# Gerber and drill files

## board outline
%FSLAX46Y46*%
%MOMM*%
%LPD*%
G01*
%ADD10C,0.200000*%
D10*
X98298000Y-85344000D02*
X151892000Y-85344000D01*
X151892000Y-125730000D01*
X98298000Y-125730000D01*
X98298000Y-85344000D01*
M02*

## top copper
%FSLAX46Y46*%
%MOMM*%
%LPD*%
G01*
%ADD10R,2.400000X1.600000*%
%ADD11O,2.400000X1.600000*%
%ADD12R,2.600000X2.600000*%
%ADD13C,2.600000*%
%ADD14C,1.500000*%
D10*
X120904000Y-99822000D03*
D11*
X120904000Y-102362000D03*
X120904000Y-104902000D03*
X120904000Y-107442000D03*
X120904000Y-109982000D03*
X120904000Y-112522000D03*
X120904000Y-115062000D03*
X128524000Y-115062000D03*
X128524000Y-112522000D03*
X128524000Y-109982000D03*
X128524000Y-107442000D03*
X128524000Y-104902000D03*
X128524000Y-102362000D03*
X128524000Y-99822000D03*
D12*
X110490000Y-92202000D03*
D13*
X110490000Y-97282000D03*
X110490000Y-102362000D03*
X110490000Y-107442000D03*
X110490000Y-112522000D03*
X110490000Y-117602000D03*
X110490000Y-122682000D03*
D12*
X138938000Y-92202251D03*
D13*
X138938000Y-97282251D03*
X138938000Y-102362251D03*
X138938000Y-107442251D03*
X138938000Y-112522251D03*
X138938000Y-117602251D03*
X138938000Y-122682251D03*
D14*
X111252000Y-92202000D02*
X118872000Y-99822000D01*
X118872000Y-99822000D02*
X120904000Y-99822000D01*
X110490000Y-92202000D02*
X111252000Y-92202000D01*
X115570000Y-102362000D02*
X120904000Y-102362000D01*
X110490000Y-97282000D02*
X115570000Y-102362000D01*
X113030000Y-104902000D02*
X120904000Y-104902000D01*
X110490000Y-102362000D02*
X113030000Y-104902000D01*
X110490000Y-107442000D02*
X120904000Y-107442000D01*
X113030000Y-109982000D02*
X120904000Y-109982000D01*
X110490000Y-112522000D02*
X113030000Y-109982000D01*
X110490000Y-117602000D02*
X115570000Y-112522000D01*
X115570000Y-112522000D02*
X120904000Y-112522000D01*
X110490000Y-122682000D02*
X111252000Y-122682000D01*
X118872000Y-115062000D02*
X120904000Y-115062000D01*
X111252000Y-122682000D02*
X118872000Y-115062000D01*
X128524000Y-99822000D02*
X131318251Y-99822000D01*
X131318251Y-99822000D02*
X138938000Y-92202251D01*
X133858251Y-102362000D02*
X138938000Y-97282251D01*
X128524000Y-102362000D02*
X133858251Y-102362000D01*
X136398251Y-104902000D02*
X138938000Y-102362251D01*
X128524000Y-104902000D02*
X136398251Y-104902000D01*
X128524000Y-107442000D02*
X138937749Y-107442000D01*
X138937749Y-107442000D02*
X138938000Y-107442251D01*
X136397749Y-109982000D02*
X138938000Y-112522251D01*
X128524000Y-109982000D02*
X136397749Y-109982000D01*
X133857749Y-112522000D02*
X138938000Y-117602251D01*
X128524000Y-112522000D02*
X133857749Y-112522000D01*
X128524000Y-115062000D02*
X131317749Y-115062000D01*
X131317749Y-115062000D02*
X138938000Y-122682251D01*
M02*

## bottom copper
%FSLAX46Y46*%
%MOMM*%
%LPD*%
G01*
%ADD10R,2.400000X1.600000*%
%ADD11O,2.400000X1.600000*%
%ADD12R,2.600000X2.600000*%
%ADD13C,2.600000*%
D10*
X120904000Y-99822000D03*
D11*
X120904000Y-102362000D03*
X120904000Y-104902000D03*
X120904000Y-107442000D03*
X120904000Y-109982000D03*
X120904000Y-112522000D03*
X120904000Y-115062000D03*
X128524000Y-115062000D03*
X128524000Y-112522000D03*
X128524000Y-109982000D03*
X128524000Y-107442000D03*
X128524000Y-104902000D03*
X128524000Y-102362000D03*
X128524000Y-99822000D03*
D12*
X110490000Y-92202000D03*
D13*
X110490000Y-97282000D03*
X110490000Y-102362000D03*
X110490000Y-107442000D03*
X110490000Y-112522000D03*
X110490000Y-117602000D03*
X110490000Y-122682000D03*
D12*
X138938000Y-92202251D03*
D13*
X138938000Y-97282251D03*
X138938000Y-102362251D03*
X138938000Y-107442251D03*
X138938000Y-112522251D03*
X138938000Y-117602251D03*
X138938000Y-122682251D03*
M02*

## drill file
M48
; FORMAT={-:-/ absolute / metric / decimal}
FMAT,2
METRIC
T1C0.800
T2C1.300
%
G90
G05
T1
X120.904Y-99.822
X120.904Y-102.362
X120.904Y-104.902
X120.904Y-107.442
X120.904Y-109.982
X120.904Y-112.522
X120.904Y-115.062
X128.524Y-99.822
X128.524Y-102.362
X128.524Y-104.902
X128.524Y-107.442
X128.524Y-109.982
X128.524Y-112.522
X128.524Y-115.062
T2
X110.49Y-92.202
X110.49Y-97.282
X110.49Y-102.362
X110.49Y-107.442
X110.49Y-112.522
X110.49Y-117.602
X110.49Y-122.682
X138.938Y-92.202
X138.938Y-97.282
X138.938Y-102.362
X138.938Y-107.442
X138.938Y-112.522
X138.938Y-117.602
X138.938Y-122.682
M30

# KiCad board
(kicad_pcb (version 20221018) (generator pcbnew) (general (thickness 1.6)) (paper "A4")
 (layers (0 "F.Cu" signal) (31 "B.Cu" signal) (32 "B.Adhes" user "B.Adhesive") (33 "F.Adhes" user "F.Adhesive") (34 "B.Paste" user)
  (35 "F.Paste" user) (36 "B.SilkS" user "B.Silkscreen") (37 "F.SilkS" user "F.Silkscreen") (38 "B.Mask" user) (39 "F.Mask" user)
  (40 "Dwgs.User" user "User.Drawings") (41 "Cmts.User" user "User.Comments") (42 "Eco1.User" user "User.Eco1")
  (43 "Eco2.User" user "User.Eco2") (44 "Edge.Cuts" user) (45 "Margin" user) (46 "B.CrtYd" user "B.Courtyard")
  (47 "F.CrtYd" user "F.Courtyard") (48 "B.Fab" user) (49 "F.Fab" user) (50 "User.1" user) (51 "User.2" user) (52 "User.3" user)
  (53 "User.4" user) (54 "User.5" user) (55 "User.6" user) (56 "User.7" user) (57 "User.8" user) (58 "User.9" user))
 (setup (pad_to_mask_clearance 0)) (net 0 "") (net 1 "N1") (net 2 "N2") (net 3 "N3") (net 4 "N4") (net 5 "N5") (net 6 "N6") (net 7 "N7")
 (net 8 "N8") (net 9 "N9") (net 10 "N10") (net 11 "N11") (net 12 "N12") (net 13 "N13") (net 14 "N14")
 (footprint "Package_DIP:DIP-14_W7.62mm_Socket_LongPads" (layer "F.Cu") (at 120.904 99.822)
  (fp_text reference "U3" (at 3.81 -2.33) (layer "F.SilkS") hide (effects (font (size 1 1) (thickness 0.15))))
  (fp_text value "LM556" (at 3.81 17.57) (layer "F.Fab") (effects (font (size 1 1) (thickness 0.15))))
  (pad "1" thru_hole rect (at 0 0) (size 2.4 1.6) (drill 0.8) (layers "*.Cu" "*.Mask") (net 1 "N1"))
  (pad "2" thru_hole oval (at 0 2.54) (size 2.4 1.6) (drill 0.8) (layers "*.Cu" "*.Mask") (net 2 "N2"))
  (pad "3" thru_hole oval (at 0 5.08) (size 2.4 1.6) (drill 0.8) (layers "*.Cu" "*.Mask") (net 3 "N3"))
  (pad "4" thru_hole oval (at 0 7.62) (size 2.4 1.6) (drill 0.8) (layers "*.Cu" "*.Mask") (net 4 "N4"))
  (pad "5" thru_hole oval (at 0 10.16) (size 2.4 1.6) (drill 0.8) (layers "*.Cu" "*.Mask") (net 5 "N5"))
  (pad "6" thru_hole oval (at 0 12.7) (size 2.4 1.6) (drill 0.8) (layers "*.Cu" "*.Mask") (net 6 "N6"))
  (pad "7" thru_hole oval (at 0 15.24) (size 2.4 1.6) (drill 0.8) (layers "*.Cu" "*.Mask") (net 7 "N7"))
  (pad "8" thru_hole oval (at 7.62 15.24) (size 2.4 1.6) (drill 0.8) (layers "*.Cu" "*.Mask") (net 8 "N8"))
  (pad "9" thru_hole oval (at 7.62 12.7) (size 2.4 1.6) (drill 0.8) (layers "*.Cu" "*.Mask") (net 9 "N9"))
  (pad "10" thru_hole oval (at 7.62 10.16) (size 2.4 1.6) (drill 0.8) (layers "*.Cu" "*.Mask") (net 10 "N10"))
  (pad "11" thru_hole oval (at 7.62 7.62) (size 2.4 1.6) (drill 0.8) (layers "*.Cu" "*.Mask") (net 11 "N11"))
  (pad "12" thru_hole oval (at 7.62 5.08) (size 2.4 1.6) (drill 0.8) (layers "*.Cu" "*.Mask") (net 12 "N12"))
  (pad "13" thru_hole oval (at 7.62 2.54) (size 2.4 1.6) (drill 0.8) (layers "*.Cu" "*.Mask") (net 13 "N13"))
  (pad "14" thru_hole oval (at 7.62 0) (size 2.4 1.6) (drill 0.8) (layers "*.Cu" "*.Mask") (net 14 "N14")))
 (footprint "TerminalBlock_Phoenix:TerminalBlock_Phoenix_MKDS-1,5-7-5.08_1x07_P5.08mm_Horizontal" (layer "F.Cu") (at 110.49 92.202 -90)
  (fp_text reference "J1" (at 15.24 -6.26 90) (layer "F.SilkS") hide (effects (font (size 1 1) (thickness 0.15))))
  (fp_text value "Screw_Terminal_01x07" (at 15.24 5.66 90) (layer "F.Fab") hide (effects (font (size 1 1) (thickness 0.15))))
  (pad "1" thru_hole rect (at 0 0 270) (size 2.6 2.6) (drill 1.3) (layers "*.Cu" "*.Mask") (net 1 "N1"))
  (pad "2" thru_hole circle (at 5.08 0 270) (size 2.6 2.6) (drill 1.3) (layers "*.Cu" "*.Mask") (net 2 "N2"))
  (pad "3" thru_hole circle (at 10.16 0 270) (size 2.6 2.6) (drill 1.3) (layers "*.Cu" "*.Mask") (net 3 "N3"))
  (pad "4" thru_hole circle (at 15.24 0 270) (size 2.6 2.6) (drill 1.3) (layers "*.Cu" "*.Mask") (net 4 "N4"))
  (pad "5" thru_hole circle (at 20.32 0 270) (size 2.6 2.6) (drill 1.3) (layers "*.Cu" "*.Mask") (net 5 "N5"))
  (pad "6" thru_hole circle (at 25.4 0 270) (size 2.6 2.6) (drill 1.3) (layers "*.Cu" "*.Mask") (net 6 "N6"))
  (pad "7" thru_hole circle (at 30.48 0 270) (size 2.6 2.6) (drill 1.3) (layers "*.Cu" "*.Mask") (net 7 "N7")))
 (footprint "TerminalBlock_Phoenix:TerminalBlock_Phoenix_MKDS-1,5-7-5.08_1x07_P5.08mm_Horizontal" (layer "F.Cu") (at 138.938 92.202251 -90)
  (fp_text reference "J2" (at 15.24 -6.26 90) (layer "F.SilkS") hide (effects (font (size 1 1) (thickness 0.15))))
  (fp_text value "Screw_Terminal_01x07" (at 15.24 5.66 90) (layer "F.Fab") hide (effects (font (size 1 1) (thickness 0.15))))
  (pad "1" thru_hole rect (at 0 0 270) (size 2.6 2.6) (drill 1.3) (layers "*.Cu" "*.Mask") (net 14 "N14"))
  (pad "2" thru_hole circle (at 5.08 0 270) (size 2.6 2.6) (drill 1.3) (layers "*.Cu" "*.Mask") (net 13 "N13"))
  (pad "3" thru_hole circle (at 10.16 0 270) (size 2.6 2.6) (drill 1.3) (layers "*.Cu" "*.Mask") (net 12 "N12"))
  (pad "4" thru_hole circle (at 15.24 0 270) (size 2.6 2.6) (drill 1.3) (layers "*.Cu" "*.Mask") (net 11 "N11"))
  (pad "5" thru_hole circle (at 20.32 0 270) (size 2.6 2.6) (drill 1.3) (layers "*.Cu" "*.Mask") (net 10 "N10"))
  (pad "6" thru_hole circle (at 25.4 0 270) (size 2.6 2.6) (drill 1.3) (layers "*.Cu" "*.Mask") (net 9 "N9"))
  (pad "7" thru_hole circle (at 30.48 0 270) (size 2.6 2.6) (drill 1.3) (layers "*.Cu" "*.Mask") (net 8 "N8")))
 (gr_rect (start 98.298 85.344) (end 151.892 125.73) (stroke (width 0.2) (type default)) (fill none) (layer "Edge.Cuts"))
 (segment (start 111.252 92.202) (end 118.872 99.822) (width 1.5) (layer "F.Cu") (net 1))
 (segment (start 118.872 99.822) (end 120.904 99.822) (width 1.5) (layer "F.Cu") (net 1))
 (segment (start 110.49 92.202) (end 111.252 92.202) (width 1.5) (layer "F.Cu") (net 1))
 (segment (start 115.57 102.362) (end 120.904 102.362) (width 1.5) (layer "F.Cu") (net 2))
 (segment (start 110.49 97.282) (end 115.57 102.362) (width 1.5) (layer "F.Cu") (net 2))
 (segment (start 113.03 104.902) (end 120.904 104.902) (width 1.5) (layer "F.Cu") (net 3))
 (segment (start 110.49 102.362) (end 113.03 104.902) (width 1.5) (layer "F.Cu") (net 3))
 (segment (start 110.49 107.442) (end 120.904 107.442) (width 1.5) (layer "F.Cu") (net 4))
 (segment (start 113.03 109.982) (end 120.904 109.982) (width 1.5) (layer "F.Cu") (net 5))
 (segment (start 110.49 112.522) (end 113.03 109.982) (width 1.5) (layer "F.Cu") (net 5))
 (segment (start 110.49 117.602) (end 115.57 112.522) (width 1.5) (layer "F.Cu") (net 6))
 (segment (start 115.57 112.522) (end 120.904 112.522) (width 1.5) (layer "F.Cu") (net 6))
 (segment (start 110.49 122.682) (end 111.252 122.682) (width 1.5) (layer "F.Cu") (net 7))
 (segment (start 118.872 115.062) (end 120.904 115.062) (width 1.5) (layer "F.Cu") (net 7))
 (segment (start 111.252 122.682) (end 118.872 115.062) (width 1.5) (layer "F.Cu") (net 7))
 (segment (start 128.524 99.822) (end 131.318251 99.822) (width 1.5) (layer "F.Cu") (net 14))
 (segment (start 131.318251 99.822) (end 138.938 92.202251) (width 1.5) (layer "F.Cu") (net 14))
 (segment (start 133.858251 102.362) (end 138.938 97.282251) (width 1.5) (layer "F.Cu") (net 13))
 (segment (start 128.524 102.362) (end 133.858251 102.362) (width 1.5) (layer "F.Cu") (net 13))
 (segment (start 136.398251 104.902) (end 138.938 102.362251) (width 1.5) (layer "F.Cu") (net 12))
 (segment (start 128.524 104.902) (end 136.398251 104.902) (width 1.5) (layer "F.Cu") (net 12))
 (segment (start 128.524 107.442) (end 138.937749 107.442) (width 1.5) (layer "F.Cu") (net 11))
 (segment (start 138.937749 107.442) (end 138.938 107.442251) (width 1.5) (layer "F.Cu") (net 11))
 (segment (start 136.397749 109.982) (end 138.938 112.522251) (width 1.5) (layer "F.Cu") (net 10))
 (segment (start 128.524 109.982) (end 136.397749 109.982) (width 1.5) (layer "F.Cu") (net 10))
 (segment (start 133.857749 112.522) (end 138.938 117.602251) (width 1.5) (layer "F.Cu") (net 9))
 (segment (start 128.524 112.522) (end 133.857749 112.522) (width 1.5) (layer "F.Cu") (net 9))
 (segment (start 128.524 115.062) (end 131.317749 115.062) (width 1.5) (layer "F.Cu") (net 8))
 (segment (start 131.317749 115.062) (end 138.938 122.682251) (width 1.5) (layer "F.Cu") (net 8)))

